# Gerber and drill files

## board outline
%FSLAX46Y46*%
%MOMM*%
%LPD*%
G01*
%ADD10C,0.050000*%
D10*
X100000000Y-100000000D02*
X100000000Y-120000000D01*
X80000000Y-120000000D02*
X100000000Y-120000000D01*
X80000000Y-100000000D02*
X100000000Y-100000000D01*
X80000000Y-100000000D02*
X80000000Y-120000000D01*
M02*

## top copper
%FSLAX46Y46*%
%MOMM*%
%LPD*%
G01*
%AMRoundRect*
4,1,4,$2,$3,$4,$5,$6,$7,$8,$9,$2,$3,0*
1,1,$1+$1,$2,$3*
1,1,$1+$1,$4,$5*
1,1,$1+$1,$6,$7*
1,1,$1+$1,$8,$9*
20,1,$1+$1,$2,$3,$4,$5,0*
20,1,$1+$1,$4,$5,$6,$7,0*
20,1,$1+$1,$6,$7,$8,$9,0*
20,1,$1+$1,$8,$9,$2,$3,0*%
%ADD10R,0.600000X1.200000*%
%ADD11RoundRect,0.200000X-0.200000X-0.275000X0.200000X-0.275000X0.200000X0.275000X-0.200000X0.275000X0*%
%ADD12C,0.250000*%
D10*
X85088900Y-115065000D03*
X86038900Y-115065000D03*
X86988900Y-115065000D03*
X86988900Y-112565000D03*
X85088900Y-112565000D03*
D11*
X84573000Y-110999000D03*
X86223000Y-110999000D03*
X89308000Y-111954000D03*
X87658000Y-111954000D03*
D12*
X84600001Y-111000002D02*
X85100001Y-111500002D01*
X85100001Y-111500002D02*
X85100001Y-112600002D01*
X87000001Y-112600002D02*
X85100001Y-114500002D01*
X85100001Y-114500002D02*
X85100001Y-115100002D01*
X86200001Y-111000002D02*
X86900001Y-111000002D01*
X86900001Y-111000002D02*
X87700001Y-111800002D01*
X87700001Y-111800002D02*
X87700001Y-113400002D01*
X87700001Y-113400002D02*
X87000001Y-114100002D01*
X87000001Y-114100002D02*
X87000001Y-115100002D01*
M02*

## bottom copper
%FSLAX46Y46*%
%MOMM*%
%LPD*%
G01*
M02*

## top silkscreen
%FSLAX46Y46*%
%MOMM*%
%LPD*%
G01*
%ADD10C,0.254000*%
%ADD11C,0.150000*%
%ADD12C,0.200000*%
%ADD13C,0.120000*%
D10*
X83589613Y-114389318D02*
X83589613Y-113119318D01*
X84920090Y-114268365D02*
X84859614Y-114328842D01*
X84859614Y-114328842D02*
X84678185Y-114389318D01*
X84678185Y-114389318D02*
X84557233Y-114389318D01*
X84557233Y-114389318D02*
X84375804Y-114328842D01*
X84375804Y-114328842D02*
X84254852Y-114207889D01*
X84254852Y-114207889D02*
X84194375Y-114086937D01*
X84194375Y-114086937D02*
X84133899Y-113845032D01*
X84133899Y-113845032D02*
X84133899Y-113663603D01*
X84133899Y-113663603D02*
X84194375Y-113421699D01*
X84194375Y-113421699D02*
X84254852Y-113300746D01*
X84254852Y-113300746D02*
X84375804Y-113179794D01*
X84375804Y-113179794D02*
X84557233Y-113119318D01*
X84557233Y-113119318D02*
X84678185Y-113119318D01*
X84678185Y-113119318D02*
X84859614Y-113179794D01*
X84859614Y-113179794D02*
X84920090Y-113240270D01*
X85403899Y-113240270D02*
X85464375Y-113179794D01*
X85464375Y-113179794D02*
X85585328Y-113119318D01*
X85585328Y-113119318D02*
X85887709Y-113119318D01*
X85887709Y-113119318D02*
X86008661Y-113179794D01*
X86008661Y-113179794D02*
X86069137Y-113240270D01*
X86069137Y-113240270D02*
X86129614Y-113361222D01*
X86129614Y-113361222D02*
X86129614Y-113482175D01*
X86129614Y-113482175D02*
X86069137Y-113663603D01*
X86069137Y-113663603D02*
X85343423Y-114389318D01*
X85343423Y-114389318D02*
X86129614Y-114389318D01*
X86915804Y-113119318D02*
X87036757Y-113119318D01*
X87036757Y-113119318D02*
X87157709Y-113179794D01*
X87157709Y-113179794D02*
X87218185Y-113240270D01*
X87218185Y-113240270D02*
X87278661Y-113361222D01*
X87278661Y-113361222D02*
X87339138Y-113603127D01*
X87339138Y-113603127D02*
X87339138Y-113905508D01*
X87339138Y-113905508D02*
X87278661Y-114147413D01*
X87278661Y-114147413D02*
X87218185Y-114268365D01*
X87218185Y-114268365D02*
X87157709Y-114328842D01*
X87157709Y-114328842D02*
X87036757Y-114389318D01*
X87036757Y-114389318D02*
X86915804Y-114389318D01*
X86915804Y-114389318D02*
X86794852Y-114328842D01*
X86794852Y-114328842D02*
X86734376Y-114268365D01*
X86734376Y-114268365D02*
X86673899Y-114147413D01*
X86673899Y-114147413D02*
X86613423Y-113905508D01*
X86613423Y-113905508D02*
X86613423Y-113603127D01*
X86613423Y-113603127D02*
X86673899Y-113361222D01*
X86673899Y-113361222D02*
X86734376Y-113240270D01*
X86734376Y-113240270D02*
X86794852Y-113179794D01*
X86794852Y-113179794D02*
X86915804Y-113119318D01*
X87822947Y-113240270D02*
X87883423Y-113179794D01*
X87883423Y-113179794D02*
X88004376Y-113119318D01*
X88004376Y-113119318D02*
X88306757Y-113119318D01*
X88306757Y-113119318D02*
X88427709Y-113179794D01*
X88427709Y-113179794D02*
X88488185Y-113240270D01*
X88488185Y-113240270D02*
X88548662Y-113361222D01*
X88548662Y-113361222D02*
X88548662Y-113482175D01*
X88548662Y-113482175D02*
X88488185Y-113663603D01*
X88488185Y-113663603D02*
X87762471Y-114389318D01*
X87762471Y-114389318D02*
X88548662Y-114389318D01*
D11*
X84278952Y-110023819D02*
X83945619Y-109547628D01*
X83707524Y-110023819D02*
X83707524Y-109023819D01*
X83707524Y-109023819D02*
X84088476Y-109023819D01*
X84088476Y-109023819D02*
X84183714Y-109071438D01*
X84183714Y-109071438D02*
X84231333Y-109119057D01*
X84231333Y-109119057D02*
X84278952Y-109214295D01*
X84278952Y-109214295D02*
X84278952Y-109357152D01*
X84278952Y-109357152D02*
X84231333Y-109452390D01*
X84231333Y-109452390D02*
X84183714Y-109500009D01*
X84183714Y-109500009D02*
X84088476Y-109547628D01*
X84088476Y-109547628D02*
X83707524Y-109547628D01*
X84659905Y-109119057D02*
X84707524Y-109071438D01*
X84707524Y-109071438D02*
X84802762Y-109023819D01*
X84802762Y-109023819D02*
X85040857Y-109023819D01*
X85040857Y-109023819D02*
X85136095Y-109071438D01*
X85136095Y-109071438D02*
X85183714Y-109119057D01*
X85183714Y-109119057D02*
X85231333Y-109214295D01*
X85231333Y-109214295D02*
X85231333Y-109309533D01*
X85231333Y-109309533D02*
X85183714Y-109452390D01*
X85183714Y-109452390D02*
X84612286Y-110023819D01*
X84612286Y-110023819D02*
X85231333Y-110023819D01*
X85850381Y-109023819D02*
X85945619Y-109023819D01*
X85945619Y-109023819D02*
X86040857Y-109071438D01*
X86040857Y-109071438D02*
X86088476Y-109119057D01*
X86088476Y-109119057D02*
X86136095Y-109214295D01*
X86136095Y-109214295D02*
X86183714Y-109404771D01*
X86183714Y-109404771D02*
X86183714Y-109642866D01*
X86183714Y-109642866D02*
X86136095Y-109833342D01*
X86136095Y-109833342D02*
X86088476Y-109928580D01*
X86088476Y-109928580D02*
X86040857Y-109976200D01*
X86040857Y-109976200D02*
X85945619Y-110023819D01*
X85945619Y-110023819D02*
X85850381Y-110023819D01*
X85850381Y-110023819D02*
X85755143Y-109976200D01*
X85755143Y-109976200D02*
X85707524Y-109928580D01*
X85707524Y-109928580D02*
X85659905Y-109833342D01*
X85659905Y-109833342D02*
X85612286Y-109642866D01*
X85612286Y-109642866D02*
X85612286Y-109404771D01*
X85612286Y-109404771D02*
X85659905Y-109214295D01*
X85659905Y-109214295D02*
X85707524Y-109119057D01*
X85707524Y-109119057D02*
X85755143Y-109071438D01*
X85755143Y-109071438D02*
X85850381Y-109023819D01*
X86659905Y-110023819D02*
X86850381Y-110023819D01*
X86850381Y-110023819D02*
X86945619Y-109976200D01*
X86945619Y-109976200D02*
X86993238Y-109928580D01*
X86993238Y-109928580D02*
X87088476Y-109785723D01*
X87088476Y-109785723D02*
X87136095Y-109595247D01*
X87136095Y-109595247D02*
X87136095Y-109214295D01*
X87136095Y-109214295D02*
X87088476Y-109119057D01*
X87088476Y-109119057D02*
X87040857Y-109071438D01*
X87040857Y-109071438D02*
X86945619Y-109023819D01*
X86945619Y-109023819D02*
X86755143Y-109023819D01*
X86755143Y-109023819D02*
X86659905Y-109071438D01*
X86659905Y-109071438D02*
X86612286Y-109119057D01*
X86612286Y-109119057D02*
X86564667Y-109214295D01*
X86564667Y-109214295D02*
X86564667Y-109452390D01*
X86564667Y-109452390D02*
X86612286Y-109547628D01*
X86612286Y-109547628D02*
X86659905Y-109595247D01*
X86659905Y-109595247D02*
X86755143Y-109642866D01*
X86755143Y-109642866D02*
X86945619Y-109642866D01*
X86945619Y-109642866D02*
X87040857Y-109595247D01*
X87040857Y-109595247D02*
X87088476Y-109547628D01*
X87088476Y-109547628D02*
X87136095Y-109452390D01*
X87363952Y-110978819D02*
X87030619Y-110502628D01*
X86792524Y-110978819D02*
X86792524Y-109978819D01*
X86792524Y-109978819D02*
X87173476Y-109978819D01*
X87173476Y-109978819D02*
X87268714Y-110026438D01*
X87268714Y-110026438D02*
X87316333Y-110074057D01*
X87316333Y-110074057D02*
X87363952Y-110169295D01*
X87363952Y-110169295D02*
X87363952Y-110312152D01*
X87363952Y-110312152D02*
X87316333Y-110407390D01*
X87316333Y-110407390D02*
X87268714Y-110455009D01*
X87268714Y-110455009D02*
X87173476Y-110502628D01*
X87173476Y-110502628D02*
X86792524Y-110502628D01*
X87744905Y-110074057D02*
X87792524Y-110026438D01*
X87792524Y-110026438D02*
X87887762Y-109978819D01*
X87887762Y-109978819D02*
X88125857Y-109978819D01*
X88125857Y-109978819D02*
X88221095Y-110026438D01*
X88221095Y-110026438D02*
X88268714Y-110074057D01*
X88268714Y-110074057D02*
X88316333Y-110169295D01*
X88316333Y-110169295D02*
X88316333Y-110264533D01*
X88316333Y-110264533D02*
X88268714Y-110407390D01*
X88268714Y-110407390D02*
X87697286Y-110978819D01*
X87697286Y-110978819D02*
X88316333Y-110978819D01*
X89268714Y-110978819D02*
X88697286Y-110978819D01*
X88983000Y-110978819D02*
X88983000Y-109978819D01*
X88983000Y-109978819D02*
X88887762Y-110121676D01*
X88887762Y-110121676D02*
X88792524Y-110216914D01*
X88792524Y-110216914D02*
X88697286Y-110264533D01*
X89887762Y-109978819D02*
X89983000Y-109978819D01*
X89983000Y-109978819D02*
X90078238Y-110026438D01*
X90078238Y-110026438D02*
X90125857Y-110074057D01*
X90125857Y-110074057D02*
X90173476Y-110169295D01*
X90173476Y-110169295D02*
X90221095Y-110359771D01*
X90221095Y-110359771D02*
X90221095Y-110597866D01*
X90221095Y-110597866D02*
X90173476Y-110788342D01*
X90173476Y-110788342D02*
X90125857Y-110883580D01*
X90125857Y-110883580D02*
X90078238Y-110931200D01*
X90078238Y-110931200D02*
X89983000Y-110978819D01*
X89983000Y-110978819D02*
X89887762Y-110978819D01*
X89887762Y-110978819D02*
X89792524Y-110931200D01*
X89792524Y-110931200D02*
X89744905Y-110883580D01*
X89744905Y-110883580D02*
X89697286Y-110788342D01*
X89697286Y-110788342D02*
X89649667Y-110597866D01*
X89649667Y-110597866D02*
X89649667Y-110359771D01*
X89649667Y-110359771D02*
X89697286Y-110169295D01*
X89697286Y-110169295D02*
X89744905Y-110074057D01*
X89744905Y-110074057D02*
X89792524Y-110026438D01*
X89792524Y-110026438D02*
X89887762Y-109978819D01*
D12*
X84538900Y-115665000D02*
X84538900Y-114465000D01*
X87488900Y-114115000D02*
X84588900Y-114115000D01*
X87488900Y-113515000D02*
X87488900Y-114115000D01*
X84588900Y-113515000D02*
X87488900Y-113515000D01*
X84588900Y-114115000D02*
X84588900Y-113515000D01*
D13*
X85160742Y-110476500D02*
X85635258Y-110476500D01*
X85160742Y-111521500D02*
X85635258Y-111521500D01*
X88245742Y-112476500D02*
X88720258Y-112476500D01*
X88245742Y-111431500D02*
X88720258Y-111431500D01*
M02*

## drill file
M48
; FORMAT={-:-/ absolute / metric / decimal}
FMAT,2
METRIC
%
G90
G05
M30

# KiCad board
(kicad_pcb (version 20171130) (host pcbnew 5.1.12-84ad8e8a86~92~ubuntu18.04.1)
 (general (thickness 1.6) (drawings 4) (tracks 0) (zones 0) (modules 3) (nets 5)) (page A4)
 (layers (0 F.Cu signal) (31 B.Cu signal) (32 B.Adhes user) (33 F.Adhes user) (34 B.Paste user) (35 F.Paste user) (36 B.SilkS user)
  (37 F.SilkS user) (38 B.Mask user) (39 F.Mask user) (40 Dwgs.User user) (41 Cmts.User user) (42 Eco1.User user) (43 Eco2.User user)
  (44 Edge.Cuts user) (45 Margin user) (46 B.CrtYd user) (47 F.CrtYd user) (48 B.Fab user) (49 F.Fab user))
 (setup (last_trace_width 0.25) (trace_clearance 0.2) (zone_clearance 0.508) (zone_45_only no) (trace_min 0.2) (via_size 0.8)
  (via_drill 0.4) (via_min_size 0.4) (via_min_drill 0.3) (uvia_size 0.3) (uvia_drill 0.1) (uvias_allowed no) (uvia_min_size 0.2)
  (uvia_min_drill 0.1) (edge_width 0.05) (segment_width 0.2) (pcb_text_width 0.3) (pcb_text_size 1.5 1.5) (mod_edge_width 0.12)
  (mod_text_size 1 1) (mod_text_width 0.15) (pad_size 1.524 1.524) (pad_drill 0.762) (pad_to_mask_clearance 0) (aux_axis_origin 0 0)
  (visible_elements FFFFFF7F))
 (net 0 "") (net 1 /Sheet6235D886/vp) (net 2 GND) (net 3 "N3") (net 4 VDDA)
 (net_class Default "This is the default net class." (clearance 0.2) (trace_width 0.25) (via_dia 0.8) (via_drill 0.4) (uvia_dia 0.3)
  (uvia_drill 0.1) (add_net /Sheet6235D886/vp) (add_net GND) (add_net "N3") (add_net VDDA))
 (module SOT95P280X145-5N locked (layer F.Cu) (at 86.038900 113.815000 90.000000)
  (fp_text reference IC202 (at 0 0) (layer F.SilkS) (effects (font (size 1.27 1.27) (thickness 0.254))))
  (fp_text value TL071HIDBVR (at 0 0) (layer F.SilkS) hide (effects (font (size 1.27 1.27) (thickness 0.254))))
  (fp_line (start -1.85 -1.5) (end -0.65 -1.5) (layer F.SilkS) (width 0.2))
  (fp_line (start -0.3 1.45) (end -0.3 -1.45) (layer F.SilkS) (width 0.2))
  (fp_line (start 0.3 1.45) (end -0.3 1.45) (layer F.SilkS) (width 0.2))
  (fp_line (start 0.3 -1.45) (end 0.3 1.45) (layer F.SilkS) (width 0.2))
  (fp_line (start -0.3 -1.45) (end 0.3 -1.45) (layer F.SilkS) (width 0.2))
  (pad 1 smd rect (at -1.25 -0.95 180.000000) (size 0.6 1.2) (layers F.Cu F.Mask F.Paste) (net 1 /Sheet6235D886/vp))
  (pad 2 smd rect (at -1.25 0 180.000000) (size 0.6 1.2) (layers F.Cu F.Mask F.Paste) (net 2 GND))
  (pad 3 smd rect (at -1.25 0.95 180.000000) (size 0.6 1.2) (layers F.Cu F.Mask F.Paste) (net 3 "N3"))
  (pad 4 smd rect (at 1.25 0.95 180.000000) (size 0.6 1.2) (layers F.Cu F.Mask F.Paste) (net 1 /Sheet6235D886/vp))
  (pad 5 smd rect (at 1.25 -0.95 180.000000) (size 0.6 1.2) (layers F.Cu F.Mask F.Paste) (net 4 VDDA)))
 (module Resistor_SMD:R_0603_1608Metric (layer F.Cu) (at 85.398000 110.999000)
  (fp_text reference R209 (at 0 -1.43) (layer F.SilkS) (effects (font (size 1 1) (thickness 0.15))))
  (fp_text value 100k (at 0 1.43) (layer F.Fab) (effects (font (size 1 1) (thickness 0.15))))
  (fp_line (start -0.237258 -0.5225) (end 0.237258 -0.5225) (layer F.SilkS) (width 0.12))
  (fp_line (start -0.237258 0.5225) (end 0.237258 0.5225) (layer F.SilkS) (width 0.12))
  (pad 1 smd roundrect (at -0.825 0) (size 0.8 0.95) (layers F.Cu F.Mask F.Paste) (roundrect_rratio 0.25) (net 4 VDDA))
  (pad 2 smd roundrect (at 0.825 0) (size 0.8 0.95) (layers F.Cu F.Mask F.Paste) (roundrect_rratio 0.25) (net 3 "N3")))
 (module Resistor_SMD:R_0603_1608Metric (layer F.Cu) (at 88.483000 111.954000)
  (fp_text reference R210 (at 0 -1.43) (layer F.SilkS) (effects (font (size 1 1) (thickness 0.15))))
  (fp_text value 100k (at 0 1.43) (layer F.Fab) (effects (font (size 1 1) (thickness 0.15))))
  (fp_line (start -0.237258 0.5225) (end 0.237258 0.5225) (layer F.SilkS) (width 0.12))
  (fp_line (start -0.237258 -0.5225) (end 0.237258 -0.5225) (layer F.SilkS) (width 0.12))
  (pad 2 smd roundrect (at 0.825 0) (size 0.8 0.95) (layers F.Cu F.Mask F.Paste) (roundrect_rratio 0.25) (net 2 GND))
  (pad 1 smd roundrect (at -0.825 0) (size 0.8 0.95) (layers F.Cu F.Mask F.Paste) (roundrect_rratio 0.25) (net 3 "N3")))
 (gr_line (start 100 100) (end 100 120) (layer Edge.Cuts) (width 0.05))
 (gr_line (start 80 120) (end 100 120) (layer Edge.Cuts) (width 0.05))
 (gr_line (start 80 100) (end 100 100) (layer Edge.Cuts) (width 0.05))
 (gr_line (start 80 100) (end 80 120) (layer Edge.Cuts) (width 0.05))
 (segment (start 84.600001 111.000002) (end 85.100001 111.500002) (width 0.250000) (layer F.Cu) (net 4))
 (segment (start 85.100001 111.500002) (end 85.100001 112.600002) (width 0.250000) (layer F.Cu) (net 4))
 (segment (start 87.000001 112.600002) (end 85.100001 114.500002) (width 0.250000) (layer F.Cu) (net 1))
 (segment (start 85.100001 114.500002) (end 85.100001 115.100002) (width 0.250000) (layer F.Cu) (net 1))
 (segment (start 86.200001 111.000002) (end 86.900001 111.000002) (width 0.250000) (layer F.Cu) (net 3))
 (segment (start 86.900001 111.000002) (end 87.700001 111.800002) (width 0.250000) (layer F.Cu) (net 3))
 (segment (start 87.700001 111.800002) (end 87.700001 113.400002) (width 0.250000) (layer F.Cu) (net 3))
 (segment (start 87.700001 113.400002) (end 87.000001 114.100002) (width 0.250000) (layer F.Cu) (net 3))
 (segment (start 87.000001 114.100002) (end 87.000001 115.100002) (width 0.250000) (layer F.Cu) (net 3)))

